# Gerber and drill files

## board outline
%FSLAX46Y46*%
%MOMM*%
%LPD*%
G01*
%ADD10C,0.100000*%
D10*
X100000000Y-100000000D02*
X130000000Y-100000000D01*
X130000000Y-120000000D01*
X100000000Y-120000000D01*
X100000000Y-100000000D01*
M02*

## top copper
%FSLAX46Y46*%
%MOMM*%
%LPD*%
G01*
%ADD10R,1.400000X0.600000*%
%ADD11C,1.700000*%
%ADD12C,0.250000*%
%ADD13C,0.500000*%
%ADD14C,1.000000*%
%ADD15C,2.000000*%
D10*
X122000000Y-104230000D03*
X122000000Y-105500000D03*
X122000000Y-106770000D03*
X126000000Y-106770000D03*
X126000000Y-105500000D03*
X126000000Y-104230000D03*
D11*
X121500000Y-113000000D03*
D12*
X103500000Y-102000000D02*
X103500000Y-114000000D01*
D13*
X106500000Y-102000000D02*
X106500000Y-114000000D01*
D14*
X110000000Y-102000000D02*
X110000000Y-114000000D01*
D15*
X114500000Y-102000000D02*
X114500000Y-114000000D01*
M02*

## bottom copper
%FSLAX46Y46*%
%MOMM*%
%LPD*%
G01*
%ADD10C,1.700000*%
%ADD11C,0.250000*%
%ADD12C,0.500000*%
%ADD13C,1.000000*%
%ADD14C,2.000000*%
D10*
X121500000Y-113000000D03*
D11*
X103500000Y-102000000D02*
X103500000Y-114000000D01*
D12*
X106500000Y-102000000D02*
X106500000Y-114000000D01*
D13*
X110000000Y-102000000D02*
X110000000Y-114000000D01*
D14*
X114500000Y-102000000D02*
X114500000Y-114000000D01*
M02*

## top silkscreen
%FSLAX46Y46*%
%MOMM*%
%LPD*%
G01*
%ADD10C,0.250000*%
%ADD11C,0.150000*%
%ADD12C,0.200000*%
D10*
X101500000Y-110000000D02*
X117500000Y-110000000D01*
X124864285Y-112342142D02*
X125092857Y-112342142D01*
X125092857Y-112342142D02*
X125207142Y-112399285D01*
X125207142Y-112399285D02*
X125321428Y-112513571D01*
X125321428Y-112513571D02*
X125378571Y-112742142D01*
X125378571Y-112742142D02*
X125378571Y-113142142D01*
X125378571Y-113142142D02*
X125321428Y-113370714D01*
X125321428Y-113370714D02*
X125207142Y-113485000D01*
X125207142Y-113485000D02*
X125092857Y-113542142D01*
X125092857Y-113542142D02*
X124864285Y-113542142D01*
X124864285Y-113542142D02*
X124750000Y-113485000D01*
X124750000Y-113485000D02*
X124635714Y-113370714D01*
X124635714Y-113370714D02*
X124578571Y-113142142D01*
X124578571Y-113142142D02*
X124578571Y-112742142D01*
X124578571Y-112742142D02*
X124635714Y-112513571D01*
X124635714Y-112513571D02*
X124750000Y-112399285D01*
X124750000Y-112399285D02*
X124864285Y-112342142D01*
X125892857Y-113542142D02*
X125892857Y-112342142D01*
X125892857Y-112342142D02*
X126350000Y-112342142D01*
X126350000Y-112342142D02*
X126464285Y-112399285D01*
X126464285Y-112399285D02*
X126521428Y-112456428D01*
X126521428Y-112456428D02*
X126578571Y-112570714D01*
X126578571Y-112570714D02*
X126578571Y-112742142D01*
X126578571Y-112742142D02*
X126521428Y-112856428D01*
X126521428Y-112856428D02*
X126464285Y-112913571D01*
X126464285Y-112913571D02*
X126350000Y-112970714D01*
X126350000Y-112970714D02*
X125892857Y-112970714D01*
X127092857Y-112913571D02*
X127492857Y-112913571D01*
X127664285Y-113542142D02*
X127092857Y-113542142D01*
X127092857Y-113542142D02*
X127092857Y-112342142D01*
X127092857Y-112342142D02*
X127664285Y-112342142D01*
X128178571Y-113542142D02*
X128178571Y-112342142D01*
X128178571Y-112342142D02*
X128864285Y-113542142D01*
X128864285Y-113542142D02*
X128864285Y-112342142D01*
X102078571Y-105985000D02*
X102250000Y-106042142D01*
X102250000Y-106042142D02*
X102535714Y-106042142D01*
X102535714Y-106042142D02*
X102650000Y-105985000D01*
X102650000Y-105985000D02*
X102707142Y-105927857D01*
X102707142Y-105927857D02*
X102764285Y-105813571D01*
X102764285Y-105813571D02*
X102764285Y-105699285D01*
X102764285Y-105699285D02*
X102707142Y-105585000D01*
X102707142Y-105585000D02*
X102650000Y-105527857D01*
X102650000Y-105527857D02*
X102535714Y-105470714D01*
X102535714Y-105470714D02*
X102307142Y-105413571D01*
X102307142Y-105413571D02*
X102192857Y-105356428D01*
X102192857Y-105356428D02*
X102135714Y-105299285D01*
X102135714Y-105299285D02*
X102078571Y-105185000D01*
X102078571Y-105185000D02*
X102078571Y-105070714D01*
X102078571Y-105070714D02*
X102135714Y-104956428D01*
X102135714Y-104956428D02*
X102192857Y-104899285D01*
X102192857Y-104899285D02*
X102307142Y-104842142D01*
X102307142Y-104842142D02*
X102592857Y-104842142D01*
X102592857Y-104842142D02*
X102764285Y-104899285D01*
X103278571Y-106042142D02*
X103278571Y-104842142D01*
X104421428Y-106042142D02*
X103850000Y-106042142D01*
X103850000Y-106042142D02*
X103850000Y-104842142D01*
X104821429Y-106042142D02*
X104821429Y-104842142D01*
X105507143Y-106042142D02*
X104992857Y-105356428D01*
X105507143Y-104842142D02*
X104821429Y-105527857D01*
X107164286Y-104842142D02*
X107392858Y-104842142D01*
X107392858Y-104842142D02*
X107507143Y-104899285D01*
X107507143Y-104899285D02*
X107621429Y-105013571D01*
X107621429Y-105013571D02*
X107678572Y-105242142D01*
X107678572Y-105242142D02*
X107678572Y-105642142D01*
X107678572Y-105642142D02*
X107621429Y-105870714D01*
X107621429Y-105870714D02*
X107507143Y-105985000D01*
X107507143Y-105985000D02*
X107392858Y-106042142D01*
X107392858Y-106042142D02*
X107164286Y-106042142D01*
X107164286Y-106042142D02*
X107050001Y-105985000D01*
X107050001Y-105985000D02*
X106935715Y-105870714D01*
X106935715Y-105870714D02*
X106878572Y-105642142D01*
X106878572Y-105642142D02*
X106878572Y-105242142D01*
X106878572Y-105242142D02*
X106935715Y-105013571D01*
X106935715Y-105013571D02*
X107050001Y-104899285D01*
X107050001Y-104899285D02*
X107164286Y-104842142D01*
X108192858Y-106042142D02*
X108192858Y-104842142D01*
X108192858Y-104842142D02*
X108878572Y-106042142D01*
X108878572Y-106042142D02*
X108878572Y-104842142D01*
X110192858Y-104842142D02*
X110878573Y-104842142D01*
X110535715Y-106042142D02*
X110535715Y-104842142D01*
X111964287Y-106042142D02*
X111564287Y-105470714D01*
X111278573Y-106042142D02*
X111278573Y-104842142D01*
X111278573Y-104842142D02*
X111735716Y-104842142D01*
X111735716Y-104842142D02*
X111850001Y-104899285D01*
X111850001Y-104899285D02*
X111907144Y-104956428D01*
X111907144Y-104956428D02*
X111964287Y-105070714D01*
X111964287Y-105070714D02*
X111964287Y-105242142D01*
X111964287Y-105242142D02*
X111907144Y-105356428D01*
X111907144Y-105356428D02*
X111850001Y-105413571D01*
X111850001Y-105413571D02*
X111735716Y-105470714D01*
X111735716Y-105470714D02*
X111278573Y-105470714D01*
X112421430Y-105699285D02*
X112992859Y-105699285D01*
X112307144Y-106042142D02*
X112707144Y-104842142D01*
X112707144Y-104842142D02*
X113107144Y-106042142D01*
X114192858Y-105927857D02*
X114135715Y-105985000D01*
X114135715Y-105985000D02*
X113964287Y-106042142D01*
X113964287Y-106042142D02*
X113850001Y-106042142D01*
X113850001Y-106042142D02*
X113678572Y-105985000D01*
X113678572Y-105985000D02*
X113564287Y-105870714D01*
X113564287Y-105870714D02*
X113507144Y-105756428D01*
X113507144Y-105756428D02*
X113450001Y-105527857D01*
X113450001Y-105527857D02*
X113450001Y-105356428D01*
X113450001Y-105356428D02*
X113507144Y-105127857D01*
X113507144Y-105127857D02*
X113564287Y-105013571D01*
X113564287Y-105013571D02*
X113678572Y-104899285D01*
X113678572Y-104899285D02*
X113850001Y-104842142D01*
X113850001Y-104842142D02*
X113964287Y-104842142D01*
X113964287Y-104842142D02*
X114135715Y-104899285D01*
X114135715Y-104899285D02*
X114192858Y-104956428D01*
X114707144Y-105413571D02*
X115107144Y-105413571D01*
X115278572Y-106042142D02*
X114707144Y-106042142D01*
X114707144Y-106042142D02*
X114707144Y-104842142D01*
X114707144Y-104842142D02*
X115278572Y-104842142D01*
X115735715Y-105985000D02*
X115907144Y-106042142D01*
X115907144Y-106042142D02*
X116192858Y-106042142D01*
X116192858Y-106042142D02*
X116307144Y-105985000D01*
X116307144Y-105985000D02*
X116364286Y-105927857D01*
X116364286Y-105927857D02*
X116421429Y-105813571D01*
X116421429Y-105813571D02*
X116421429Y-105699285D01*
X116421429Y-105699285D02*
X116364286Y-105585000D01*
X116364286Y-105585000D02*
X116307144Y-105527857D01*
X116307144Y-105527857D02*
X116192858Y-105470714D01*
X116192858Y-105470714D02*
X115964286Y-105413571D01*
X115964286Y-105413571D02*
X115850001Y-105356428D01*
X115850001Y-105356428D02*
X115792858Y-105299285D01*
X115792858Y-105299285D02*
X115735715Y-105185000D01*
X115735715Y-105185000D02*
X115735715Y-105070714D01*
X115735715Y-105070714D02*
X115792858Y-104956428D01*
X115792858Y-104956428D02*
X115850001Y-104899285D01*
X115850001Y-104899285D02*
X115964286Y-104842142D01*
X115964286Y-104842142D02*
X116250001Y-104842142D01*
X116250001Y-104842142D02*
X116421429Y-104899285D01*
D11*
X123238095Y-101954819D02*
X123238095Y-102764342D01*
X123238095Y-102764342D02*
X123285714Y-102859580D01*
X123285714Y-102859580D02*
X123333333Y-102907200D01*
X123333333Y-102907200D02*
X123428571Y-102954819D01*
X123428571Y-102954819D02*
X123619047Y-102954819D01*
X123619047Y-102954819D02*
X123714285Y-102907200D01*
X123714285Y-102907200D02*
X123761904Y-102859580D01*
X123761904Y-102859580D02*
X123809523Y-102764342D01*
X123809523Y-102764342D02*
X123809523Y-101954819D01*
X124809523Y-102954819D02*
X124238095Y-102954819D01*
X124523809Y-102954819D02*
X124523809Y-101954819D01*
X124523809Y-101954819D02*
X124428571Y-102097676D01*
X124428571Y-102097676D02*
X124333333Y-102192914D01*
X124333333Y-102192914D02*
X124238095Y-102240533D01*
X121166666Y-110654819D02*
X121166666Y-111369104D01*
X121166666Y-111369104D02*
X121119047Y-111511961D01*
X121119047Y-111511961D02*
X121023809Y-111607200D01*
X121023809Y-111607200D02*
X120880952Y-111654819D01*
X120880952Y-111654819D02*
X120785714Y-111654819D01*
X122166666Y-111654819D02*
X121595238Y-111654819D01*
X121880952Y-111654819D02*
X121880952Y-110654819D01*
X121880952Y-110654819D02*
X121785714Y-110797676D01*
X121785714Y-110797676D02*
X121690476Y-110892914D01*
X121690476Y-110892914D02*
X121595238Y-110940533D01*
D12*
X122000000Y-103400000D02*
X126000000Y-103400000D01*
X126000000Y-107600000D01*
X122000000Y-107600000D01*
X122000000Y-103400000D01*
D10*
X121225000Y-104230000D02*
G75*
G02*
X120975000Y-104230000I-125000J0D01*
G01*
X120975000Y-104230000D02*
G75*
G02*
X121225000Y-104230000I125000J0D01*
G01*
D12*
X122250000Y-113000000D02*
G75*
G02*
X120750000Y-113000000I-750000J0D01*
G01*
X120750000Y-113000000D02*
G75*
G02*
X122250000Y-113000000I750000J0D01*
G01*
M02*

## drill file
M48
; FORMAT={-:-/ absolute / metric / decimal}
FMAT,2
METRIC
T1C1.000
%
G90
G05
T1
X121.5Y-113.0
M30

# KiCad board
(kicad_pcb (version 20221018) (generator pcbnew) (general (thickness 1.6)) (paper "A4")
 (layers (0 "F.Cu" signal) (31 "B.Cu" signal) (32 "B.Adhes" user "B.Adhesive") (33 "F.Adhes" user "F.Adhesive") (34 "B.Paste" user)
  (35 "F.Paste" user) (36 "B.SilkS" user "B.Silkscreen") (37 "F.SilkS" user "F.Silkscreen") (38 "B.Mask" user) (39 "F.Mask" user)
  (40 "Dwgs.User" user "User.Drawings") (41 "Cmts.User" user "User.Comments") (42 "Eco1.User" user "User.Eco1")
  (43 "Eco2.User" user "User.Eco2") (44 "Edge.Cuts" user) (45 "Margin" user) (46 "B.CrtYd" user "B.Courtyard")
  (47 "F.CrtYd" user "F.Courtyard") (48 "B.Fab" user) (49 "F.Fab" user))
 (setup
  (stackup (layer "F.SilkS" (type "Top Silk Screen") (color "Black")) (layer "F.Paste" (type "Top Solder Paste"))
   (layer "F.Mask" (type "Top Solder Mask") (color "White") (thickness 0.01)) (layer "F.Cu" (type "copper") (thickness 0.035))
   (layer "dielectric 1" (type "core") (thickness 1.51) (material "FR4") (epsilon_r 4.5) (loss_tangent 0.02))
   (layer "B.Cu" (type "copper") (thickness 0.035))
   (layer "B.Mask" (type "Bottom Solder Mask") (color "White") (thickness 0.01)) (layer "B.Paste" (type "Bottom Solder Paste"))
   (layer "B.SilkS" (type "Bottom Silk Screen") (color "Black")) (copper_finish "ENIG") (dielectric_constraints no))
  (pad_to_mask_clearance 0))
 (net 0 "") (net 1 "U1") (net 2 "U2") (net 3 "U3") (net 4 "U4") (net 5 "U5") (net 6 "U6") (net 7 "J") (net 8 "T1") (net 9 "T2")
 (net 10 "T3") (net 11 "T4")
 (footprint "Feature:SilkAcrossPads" (layer "F.Cu") (at 124 105.5)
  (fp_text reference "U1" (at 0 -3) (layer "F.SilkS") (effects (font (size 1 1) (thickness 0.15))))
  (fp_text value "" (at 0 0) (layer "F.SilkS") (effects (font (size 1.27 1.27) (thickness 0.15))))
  (fp_rect (start -2 -2.1) (end 2 2.1) (stroke (width 0.2) (type solid)) (fill none) (layer "F.SilkS"))
  (fp_circle (center -2.9 -1.27) (end -2.65 -1.27) (stroke (width 0) (type solid)) (fill solid) (layer "F.SilkS"))
  (pad "1" smd rect (at -2 -1.27) (size 1.4 0.6) (layers "F.Cu" "F.Paste" "F.Mask") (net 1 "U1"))
  (pad "2" smd rect (at -2 0) (size 1.4 0.6) (layers "F.Cu" "F.Paste" "F.Mask") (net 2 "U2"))
  (pad "3" smd rect (at -2 1.27) (size 1.4 0.6) (layers "F.Cu" "F.Paste" "F.Mask") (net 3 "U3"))
  (pad "4" smd rect (at 2 1.27) (size 1.4 0.6) (layers "F.Cu" "F.Paste" "F.Mask") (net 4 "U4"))
  (pad "5" smd rect (at 2 0) (size 1.4 0.6) (layers "F.Cu" "F.Paste" "F.Mask") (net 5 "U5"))
  (pad "6" smd rect (at 2 -1.27) (size 1.4 0.6) (layers "F.Cu" "F.Paste" "F.Mask") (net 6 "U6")))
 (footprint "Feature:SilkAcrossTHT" (layer "F.Cu") (at 121.5 113)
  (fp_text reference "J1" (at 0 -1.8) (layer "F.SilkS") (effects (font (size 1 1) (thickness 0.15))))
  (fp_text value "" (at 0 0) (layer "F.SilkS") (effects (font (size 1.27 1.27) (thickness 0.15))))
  (fp_circle (center 0 0) (end 0.75 0) (stroke (width 0.2) (type solid)) (fill none) (layer "F.SilkS"))
  (pad "1" thru_hole circle (at 0 0) (size 1.7 1.7) (drill 1) (layers "*.Cu" "*.Mask") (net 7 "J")))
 (gr_line (start 101.5 110) (end 117.5 110) (stroke (width 0.25) (type solid)) (layer "F.SilkS"))
 (gr_rect (start 100 100) (end 130 120) (stroke (width 0.1) (type solid)) (fill none) (layer "Edge.Cuts"))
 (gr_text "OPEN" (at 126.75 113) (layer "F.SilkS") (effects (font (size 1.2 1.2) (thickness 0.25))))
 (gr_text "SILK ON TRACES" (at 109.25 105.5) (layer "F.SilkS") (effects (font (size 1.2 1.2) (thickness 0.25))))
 (segment (start 103.5 102) (end 103.5 114) (width 0.25) (layer "F.Cu") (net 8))
 (segment (start 103.5 102) (end 103.5 114) (width 0.25) (layer "B.Cu") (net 8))
 (segment (start 106.5 102) (end 106.5 114) (width 0.5) (layer "F.Cu") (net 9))
 (segment (start 106.5 102) (end 106.5 114) (width 0.5) (layer "B.Cu") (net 9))
 (segment (start 110 102) (end 110 114) (width 1) (layer "F.Cu") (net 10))
 (segment (start 110 102) (end 110 114) (width 1) (layer "B.Cu") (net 10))
 (segment (start 114.5 102) (end 114.5 114) (width 2) (layer "F.Cu") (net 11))
 (segment (start 114.5 102) (end 114.5 114) (width 2) (layer "B.Cu") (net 11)))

